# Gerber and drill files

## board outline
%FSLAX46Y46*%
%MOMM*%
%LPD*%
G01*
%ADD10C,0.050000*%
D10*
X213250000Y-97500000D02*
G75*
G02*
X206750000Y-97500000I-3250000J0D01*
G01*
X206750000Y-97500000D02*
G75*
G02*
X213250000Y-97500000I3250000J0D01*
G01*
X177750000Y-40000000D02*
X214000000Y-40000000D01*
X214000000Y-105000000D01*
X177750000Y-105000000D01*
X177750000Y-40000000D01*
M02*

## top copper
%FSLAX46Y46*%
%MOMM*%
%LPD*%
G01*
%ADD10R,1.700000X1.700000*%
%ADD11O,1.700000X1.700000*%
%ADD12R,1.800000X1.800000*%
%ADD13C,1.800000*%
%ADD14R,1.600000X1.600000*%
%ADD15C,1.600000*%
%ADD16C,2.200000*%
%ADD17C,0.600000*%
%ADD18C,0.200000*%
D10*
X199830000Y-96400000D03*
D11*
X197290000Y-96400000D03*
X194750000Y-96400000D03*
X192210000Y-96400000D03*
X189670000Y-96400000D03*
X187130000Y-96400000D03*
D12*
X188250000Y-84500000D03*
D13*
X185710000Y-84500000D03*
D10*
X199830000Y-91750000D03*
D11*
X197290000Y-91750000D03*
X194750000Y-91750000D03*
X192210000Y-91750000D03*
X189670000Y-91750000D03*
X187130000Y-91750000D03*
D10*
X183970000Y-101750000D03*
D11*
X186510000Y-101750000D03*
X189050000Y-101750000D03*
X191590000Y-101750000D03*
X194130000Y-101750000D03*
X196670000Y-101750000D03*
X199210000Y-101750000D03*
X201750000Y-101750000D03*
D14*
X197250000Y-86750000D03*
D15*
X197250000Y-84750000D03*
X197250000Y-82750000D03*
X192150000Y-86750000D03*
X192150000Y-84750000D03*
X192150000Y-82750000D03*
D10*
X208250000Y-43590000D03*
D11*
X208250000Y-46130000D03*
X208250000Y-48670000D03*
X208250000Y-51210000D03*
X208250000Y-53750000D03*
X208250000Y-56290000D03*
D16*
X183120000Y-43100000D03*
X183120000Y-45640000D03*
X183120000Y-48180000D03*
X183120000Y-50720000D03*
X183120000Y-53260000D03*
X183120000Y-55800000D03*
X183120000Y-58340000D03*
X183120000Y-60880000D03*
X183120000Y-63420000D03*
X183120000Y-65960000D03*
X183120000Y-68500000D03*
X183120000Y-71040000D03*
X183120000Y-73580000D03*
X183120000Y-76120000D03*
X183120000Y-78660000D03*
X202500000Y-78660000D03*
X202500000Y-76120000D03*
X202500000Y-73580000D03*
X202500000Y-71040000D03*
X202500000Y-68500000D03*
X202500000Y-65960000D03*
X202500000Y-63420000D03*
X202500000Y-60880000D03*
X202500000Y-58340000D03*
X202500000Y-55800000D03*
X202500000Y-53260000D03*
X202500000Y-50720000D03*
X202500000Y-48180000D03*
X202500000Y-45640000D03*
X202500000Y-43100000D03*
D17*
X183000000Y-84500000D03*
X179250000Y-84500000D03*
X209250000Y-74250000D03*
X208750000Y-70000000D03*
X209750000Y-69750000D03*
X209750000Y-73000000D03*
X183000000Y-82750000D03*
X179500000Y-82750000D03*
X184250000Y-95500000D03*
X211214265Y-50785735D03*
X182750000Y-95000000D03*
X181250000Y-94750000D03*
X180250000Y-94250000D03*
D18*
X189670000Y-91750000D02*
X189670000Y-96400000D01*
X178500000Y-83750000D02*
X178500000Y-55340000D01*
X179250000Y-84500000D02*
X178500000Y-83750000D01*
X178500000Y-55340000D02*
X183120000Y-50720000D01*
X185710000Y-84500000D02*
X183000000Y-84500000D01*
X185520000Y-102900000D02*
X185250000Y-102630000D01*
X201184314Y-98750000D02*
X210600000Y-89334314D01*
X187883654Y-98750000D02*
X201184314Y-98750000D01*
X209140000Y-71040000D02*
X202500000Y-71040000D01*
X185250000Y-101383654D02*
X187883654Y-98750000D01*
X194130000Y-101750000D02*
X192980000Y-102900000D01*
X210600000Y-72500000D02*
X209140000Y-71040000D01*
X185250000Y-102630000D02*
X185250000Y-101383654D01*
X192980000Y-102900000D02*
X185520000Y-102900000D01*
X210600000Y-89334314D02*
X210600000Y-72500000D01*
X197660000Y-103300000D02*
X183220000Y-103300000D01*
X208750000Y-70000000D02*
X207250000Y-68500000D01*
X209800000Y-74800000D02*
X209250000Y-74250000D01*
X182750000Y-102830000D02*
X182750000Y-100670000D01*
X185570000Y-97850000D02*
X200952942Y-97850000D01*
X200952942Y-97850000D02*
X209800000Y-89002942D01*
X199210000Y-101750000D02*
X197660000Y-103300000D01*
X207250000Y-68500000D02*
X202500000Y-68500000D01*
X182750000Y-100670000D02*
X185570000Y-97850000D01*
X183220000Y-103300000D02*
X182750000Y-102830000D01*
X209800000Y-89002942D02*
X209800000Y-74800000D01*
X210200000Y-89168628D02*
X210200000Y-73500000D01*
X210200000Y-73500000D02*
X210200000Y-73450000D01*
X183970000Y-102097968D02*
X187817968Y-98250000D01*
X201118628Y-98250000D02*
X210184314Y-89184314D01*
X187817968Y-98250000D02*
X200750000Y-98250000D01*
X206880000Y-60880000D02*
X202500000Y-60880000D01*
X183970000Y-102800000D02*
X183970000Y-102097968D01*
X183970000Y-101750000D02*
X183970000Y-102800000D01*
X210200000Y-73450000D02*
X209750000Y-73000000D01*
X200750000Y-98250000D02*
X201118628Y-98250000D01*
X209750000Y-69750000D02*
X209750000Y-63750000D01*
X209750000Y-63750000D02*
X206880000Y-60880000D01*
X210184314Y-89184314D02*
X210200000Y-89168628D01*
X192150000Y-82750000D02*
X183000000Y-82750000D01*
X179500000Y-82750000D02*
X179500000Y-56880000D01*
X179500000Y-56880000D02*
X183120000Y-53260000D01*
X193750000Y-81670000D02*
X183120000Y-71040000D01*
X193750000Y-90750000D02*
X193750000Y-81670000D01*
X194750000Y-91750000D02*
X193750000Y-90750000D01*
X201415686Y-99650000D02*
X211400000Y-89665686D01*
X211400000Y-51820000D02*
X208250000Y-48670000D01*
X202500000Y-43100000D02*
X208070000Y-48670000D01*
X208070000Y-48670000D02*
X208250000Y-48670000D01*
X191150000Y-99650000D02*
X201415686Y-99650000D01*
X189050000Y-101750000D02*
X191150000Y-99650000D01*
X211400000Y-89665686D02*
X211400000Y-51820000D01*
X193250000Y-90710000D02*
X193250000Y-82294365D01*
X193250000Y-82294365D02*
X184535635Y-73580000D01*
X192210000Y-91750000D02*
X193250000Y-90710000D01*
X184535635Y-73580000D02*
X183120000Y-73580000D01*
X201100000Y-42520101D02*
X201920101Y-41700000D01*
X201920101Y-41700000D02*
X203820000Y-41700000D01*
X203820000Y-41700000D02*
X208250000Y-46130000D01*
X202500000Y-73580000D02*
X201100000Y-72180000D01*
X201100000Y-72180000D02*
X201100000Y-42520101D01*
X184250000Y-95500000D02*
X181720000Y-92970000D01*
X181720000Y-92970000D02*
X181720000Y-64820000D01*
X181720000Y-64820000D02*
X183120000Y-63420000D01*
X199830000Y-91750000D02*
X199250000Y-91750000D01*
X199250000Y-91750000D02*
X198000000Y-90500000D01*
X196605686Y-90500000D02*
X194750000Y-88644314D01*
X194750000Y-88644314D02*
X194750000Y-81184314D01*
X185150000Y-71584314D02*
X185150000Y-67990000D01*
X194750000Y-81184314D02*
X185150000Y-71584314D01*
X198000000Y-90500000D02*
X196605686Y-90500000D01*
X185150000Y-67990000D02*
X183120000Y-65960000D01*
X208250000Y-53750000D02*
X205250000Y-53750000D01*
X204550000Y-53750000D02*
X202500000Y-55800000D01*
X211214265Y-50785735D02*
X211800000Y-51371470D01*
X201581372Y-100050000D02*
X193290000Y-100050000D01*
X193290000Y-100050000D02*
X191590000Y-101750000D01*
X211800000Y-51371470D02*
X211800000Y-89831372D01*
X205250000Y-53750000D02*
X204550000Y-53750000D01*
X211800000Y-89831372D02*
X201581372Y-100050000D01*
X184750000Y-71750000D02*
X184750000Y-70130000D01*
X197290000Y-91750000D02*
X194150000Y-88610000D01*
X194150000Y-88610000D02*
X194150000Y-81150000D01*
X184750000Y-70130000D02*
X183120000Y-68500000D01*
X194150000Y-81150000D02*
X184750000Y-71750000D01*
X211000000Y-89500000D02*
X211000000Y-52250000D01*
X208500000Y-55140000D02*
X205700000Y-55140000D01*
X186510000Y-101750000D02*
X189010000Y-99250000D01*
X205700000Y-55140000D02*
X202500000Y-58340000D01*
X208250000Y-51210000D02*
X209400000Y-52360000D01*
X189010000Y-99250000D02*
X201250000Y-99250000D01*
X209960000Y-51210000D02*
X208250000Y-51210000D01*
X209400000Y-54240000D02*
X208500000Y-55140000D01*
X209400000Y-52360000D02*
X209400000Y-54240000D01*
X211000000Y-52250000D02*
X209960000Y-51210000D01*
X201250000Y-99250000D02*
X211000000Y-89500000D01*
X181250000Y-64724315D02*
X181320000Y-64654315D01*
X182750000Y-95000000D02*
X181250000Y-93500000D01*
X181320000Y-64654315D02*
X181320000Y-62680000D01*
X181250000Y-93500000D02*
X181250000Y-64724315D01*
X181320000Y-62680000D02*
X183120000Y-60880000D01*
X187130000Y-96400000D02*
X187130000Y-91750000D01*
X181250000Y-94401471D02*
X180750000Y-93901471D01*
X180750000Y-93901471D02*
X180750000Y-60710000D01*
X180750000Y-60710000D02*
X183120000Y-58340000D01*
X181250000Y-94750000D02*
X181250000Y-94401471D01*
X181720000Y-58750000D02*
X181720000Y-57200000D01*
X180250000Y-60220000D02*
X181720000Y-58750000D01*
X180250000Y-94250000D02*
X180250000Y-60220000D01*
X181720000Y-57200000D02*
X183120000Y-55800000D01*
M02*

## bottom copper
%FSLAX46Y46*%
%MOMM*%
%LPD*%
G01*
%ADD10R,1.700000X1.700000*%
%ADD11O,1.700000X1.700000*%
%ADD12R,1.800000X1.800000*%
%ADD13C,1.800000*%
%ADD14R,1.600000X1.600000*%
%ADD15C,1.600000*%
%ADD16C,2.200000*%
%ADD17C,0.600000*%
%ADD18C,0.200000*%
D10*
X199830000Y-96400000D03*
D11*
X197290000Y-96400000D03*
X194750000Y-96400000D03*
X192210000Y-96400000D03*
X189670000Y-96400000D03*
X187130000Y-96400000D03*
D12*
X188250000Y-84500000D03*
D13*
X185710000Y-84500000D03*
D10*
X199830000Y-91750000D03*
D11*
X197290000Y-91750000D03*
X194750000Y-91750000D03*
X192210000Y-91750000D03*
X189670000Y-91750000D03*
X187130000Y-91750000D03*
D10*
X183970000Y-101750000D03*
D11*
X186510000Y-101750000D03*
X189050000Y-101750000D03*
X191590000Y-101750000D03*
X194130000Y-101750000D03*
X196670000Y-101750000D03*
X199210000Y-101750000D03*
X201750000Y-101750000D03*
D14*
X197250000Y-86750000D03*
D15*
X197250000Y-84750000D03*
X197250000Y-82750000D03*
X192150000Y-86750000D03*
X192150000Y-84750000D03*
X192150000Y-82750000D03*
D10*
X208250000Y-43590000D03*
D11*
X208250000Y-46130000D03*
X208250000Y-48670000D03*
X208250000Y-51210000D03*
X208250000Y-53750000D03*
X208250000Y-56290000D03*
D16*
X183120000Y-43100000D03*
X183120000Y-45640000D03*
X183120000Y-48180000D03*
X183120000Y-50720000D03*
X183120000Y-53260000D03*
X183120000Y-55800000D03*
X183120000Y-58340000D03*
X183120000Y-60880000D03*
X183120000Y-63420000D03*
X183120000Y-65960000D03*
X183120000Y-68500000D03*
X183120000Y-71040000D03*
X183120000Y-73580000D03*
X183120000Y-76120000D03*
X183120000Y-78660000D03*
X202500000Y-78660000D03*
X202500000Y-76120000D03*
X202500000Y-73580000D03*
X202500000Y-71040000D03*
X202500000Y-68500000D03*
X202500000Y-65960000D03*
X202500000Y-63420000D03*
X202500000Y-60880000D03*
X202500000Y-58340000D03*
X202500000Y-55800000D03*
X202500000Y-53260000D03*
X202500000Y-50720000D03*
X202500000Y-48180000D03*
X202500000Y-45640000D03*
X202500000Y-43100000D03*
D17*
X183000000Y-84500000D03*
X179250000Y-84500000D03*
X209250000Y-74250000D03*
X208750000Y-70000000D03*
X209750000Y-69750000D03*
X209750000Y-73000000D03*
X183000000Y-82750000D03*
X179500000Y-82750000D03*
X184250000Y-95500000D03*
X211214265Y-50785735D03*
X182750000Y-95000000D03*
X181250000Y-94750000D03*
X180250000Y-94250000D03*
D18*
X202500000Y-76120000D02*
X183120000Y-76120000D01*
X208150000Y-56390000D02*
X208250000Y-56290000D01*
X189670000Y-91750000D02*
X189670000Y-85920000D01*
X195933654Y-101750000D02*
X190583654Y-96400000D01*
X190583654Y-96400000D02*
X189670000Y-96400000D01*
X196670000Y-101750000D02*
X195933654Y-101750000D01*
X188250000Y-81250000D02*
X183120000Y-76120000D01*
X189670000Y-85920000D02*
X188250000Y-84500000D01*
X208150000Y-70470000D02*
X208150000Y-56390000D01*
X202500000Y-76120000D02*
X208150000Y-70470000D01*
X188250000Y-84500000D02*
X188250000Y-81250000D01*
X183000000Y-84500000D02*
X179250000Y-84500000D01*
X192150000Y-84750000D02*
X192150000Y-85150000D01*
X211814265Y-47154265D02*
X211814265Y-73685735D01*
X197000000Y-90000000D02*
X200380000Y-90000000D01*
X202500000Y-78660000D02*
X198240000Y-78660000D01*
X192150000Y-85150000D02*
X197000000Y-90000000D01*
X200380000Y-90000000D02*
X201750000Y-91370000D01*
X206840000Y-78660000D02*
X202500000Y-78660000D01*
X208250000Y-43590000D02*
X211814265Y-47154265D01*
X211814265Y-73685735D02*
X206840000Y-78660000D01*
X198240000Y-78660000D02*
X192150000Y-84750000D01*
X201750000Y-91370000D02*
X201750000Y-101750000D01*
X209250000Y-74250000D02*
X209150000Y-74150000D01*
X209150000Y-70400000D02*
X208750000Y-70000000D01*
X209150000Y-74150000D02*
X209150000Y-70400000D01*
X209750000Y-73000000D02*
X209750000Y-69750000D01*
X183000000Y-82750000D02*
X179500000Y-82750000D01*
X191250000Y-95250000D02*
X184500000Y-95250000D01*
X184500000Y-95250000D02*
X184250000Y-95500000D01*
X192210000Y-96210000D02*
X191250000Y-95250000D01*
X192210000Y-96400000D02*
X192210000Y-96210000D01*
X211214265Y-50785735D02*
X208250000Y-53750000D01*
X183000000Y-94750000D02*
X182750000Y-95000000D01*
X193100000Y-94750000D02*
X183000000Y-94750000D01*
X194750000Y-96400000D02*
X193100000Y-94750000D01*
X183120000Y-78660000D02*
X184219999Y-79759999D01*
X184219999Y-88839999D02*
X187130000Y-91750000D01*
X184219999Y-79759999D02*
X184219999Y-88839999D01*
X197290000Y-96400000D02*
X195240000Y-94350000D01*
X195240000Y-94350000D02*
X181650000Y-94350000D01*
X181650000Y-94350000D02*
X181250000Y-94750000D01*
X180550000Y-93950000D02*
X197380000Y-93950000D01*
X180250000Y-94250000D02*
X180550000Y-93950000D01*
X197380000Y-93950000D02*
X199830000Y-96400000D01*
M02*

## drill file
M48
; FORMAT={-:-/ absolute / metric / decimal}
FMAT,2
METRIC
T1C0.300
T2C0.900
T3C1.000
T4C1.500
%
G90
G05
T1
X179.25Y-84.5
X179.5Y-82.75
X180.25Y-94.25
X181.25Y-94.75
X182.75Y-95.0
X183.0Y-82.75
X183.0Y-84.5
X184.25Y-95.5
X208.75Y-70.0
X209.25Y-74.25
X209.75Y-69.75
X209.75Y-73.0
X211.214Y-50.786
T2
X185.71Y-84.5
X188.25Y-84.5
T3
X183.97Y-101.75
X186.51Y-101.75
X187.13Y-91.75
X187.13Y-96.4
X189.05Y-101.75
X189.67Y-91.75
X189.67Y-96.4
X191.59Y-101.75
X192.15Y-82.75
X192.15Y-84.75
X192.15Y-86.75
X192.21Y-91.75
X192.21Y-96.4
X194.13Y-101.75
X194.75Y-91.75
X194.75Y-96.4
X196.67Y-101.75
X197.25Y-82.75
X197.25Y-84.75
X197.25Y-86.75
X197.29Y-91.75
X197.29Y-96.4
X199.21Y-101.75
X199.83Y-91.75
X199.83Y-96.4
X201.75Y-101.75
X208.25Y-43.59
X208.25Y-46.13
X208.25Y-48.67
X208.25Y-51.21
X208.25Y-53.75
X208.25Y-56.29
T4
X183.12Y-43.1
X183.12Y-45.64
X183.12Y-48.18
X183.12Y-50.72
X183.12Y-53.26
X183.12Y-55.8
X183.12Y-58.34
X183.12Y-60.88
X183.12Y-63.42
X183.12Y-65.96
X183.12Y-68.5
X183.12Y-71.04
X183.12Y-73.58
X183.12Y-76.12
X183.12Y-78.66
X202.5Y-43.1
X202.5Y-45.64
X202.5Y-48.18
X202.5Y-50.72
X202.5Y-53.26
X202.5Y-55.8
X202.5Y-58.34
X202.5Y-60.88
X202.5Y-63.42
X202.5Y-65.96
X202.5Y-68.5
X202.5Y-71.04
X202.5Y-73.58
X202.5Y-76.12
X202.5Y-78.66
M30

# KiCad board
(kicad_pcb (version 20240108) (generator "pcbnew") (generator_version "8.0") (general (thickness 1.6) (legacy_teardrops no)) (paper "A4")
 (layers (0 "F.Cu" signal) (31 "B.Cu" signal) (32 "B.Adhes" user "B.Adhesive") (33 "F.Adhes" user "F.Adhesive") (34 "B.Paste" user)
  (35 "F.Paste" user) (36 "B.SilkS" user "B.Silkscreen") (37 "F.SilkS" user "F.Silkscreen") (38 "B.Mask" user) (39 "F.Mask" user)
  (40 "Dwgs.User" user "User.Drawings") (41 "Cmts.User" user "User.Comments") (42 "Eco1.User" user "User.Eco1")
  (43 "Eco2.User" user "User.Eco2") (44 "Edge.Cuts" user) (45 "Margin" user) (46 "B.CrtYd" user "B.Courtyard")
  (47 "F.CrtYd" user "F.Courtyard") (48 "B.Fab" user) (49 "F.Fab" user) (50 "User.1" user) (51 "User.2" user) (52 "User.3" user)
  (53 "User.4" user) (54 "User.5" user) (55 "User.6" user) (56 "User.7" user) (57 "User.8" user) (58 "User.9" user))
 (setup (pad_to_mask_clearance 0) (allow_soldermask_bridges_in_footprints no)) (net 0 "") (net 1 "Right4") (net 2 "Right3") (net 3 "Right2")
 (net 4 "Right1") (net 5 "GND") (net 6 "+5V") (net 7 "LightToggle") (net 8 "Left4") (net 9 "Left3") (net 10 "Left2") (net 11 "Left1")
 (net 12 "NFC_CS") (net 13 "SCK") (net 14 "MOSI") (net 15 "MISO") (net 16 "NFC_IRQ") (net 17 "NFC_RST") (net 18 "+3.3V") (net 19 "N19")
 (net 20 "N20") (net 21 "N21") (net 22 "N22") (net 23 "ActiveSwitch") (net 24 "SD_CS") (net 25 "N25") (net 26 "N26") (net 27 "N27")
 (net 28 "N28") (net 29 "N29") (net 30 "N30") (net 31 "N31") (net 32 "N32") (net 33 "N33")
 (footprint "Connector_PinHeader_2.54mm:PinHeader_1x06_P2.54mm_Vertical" (layer "F.Cu") (at 199.83 96.4 -90)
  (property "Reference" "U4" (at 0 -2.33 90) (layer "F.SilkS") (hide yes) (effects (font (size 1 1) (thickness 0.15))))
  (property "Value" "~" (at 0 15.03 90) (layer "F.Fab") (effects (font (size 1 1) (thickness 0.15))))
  (pad "1" thru_hole rect (at 0 0 270) (size 1.7 1.7) (drill 1) (layers "*.Cu" "*.Mask") (remove_unused_layers no) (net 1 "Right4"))
  (pad "2" thru_hole oval (at 0 2.54 270) (size 1.7 1.7) (drill 1) (layers "*.Cu" "*.Mask") (remove_unused_layers no) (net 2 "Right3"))
  (pad "3" thru_hole oval (at 0 5.08 270) (size 1.7 1.7) (drill 1) (layers "*.Cu" "*.Mask") (remove_unused_layers no) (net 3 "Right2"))
  (pad "4" thru_hole oval (at 0 7.62 270) (size 1.7 1.7) (drill 1) (layers "*.Cu" "*.Mask") (remove_unused_layers no) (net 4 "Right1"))
  (pad "5" thru_hole oval (at 0 10.16 270) (size 1.7 1.7) (drill 1) (layers "*.Cu" "*.Mask") (remove_unused_layers no) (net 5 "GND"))
  (pad "6" thru_hole oval (at 0 12.7 270) (size 1.7 1.7) (drill 1) (layers "*.Cu" "*.Mask") (remove_unused_layers no) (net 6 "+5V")))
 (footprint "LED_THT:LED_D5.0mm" (layer "F.Cu") (at 188.25 84.5 180)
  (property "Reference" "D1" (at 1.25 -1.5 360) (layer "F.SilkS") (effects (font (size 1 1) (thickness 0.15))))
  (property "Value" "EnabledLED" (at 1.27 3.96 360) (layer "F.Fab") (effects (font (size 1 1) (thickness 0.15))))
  (pad "1" thru_hole rect (at 0 0 180) (size 1.8 1.8) (drill 0.9) (layers "*.Cu" "*.Mask") (remove_unused_layers no) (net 5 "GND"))
  (pad "2" thru_hole circle (at 2.54 0 180) (size 1.8 1.8) (drill 0.9) (layers "*.Cu" "*.Mask") (remove_unused_layers no)
   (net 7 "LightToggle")))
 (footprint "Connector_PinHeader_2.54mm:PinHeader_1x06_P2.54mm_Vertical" (layer "F.Cu") (at 199.83 91.75 -90)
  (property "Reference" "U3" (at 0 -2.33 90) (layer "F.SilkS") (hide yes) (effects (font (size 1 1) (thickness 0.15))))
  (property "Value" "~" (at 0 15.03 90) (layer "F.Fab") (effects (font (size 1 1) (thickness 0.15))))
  (pad "1" thru_hole rect (at 0 0 270) (size 1.7 1.7) (drill 1) (layers "*.Cu" "*.Mask") (remove_unused_layers no) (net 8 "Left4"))
  (pad "2" thru_hole oval (at 0 2.54 270) (size 1.7 1.7) (drill 1) (layers "*.Cu" "*.Mask") (remove_unused_layers no) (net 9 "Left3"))
  (pad "3" thru_hole oval (at 0 5.08 270) (size 1.7 1.7) (drill 1) (layers "*.Cu" "*.Mask") (remove_unused_layers no) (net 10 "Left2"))
  (pad "4" thru_hole oval (at 0 7.62 270) (size 1.7 1.7) (drill 1) (layers "*.Cu" "*.Mask") (remove_unused_layers no) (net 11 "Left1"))
  (pad "5" thru_hole oval (at 0 10.16 270) (size 1.7 1.7) (drill 1) (layers "*.Cu" "*.Mask") (remove_unused_layers no) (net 5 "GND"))
  (pad "6" thru_hole oval (at 0 12.7 270) (size 1.7 1.7) (drill 1) (layers "*.Cu" "*.Mask") (remove_unused_layers no) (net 6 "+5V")))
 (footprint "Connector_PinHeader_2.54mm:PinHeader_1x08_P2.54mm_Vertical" (layer "F.Cu") (at 183.97 101.75 90)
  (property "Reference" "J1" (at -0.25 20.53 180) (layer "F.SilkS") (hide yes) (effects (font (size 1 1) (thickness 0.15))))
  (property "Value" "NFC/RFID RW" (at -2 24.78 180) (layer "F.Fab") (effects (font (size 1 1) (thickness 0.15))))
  (pad "1" thru_hole rect (at 0 0 90) (size 1.7 1.7) (drill 1) (layers "*.Cu" "*.Mask") (remove_unused_layers no) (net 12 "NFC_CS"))
  (pad "2" thru_hole oval (at 0 2.54 90) (size 1.7 1.7) (drill 1) (layers "*.Cu" "*.Mask") (remove_unused_layers no) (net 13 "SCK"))
  (pad "3" thru_hole oval (at 0 5.08 90) (size 1.7 1.7) (drill 1) (layers "*.Cu" "*.Mask") (remove_unused_layers no) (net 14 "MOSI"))
  (pad "4" thru_hole oval (at 0 7.62 90) (size 1.7 1.7) (drill 1) (layers "*.Cu" "*.Mask") (remove_unused_layers no) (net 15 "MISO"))
  (pad "5" thru_hole oval (at 0 10.16 90) (size 1.7 1.7) (drill 1) (layers "*.Cu" "*.Mask") (remove_unused_layers no) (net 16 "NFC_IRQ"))
  (pad "6" thru_hole oval (at 0 12.7 90) (size 1.7 1.7) (drill 1) (layers "*.Cu" "*.Mask") (remove_unused_layers no) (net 5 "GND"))
  (pad "7" thru_hole oval (at 0 15.24 90) (size 1.7 1.7) (drill 1) (layers "*.Cu" "*.Mask") (remove_unused_layers no) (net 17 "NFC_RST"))
  (pad "8" thru_hole oval (at 0 17.78 90) (size 1.7 1.7) (drill 1) (layers "*.Cu" "*.Mask") (remove_unused_layers no) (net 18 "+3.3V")))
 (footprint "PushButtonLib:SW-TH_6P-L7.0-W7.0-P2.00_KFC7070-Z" (layer "F.Cu") (at 194.7 84.75)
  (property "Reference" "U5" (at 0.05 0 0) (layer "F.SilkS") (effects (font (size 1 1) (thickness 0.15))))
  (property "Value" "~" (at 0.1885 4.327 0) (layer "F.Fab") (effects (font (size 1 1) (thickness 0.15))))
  (pad "1" thru_hole rect (at 2.55 2 270) (size 1.6 1.6) (drill 1) (layers "*.Cu" "*.Mask") (remove_unused_layers no) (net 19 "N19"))
  (pad "2" thru_hole circle (at 2.55 0 270) (size 1.6 1.6) (drill 1) (layers "*.Cu" "*.Mask") (remove_unused_layers no) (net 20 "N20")
   (thermal_bridge_angle 90))
  (pad "3" thru_hole circle (at 2.55 -2 270) (size 1.6 1.6) (drill 1) (layers "*.Cu" "*.Mask") (remove_unused_layers no) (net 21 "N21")
   (thermal_bridge_angle 90))
  (pad "4" thru_hole circle (at -2.55 2 270) (size 1.6 1.6) (drill 1) (layers "*.Cu" "*.Mask") (remove_unused_layers no) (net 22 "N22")
   (thermal_bridge_angle 90))
  (pad "5" thru_hole circle (at -2.55 0 270) (size 1.6 1.6) (drill 1) (layers "*.Cu" "*.Mask") (remove_unused_layers no) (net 18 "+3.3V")
   (thermal_bridge_angle 90))
  (pad "6" thru_hole circle (at -2.55 -2 270) (size 1.6 1.6) (drill 1) (layers "*.Cu" "*.Mask") (remove_unused_layers no)
   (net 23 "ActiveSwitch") (thermal_bridge_angle 90)))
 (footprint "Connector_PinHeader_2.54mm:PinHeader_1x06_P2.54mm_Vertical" (layer "F.Cu") (at 208.25 43.59)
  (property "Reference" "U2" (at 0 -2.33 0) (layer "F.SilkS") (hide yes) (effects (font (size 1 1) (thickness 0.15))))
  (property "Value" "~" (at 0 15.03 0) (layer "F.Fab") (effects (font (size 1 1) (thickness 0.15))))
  (pad "1" thru_hole rect (at 0 0) (size 1.7 1.7) (drill 1) (layers "*.Cu" "*.Mask") (remove_unused_layers no) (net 18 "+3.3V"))
  (pad "2" thru_hole oval (at 0 2.54) (size 1.7 1.7) (drill 1) (layers "*.Cu" "*.Mask") (remove_unused_layers no) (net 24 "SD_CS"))
  (pad "3" thru_hole oval (at 0 5.08) (size 1.7 1.7) (drill 1) (layers "*.Cu" "*.Mask") (remove_unused_layers no) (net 14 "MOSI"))
  (pad "4" thru_hole oval (at 0 7.62) (size 1.7 1.7) (drill 1) (layers "*.Cu" "*.Mask") (remove_unused_layers no) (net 13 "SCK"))
  (pad "5" thru_hole oval (at 0 10.16) (size 1.7 1.7) (drill 1) (layers "*.Cu" "*.Mask") (remove_unused_layers no) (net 15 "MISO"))
  (pad "6" thru_hole oval (at 0 12.7) (size 1.7 1.7) (drill 1) (layers "*.Cu" "*.Mask") (remove_unused_layers no) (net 5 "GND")))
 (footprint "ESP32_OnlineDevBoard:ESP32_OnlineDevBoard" (layer "F.Cu") (at 192.901386 67.23 -90)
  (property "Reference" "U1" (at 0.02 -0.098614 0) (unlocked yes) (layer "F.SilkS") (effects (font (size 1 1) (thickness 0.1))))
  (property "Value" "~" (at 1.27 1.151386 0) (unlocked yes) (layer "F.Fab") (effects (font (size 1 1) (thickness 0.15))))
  (pad "1" thru_hole circle (at -24.13 9.781386 270) (size 2.2 2.2) (drill 1.5) (layers "*.Cu" "*.Mask") (remove_unused_layers no)
   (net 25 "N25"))
  (pad "2" thru_hole circle (at -21.59 9.781386 270) (size 2.2 2.2) (drill 1.5) (layers "*.Cu" "*.Mask") (remove_unused_layers no)
   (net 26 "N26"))
  (pad "3" thru_hole circle (at -19.05 9.781386 270) (size 2.2 2.2) (drill 1.5) (layers "*.Cu" "*.Mask") (remove_unused_layers no)
   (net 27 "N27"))
  (pad "4" thru_hole circle (at -16.51 9.781386 270) (size 2.2 2.2) (drill 1.5) (layers "*.Cu" "*.Mask") (remove_unused_layers no)
   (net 7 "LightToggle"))
  (pad "5" thru_hole circle (at -13.97 9.781386 270) (size 2.2 2.2) (drill 1.5) (layers "*.Cu" "*.Mask") (remove_unused_layers no)
   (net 23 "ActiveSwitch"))
  (pad "6" thru_hole circle (at -11.43 9.781386 270) (size 2.2 2.2) (drill 1.5) (layers "*.Cu" "*.Mask") (remove_unused_layers no)
   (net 1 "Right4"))
  (pad "7" thru_hole circle (at -8.89 9.781386 270) (size 2.2 2.2) (drill 1.5) (layers "*.Cu" "*.Mask") (remove_unused_layers no)
   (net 2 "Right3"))
  (pad "8" thru_hole circle (at -6.35 9.781386 270) (size 2.2 2.2) (drill 1.5) (layers "*.Cu" "*.Mask") (remove_unused_layers no)
   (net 3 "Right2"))
  (pad "9" thru_hole circle (at -3.81 9.781386 270) (size 2.2 2.2) (drill 1.5) (layers "*.Cu" "*.Mask") (remove_unused_layers no)
   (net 4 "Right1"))
  (pad "10" thru_hole circle (at -1.27 9.781386 270) (size 2.2 2.2) (drill 1.5) (layers "*.Cu" "*.Mask") (remove_unused_layers no)
   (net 8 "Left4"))
  (pad "11" thru_hole circle (at 1.27 9.781386 270) (size 2.2 2.2) (drill 1.5) (layers "*.Cu" "*.Mask") (remove_unused_layers no)
   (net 9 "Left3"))
  (pad "12" thru_hole circle (at 3.81 9.781386 270) (size 2.2 2.2) (drill 1.5) (layers "*.Cu" "*.Mask") (remove_unused_layers no)
   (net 10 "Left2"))
  (pad "13" thru_hole circle (at 6.35 9.781386 270) (size 2.2 2.2) (drill 1.5) (layers "*.Cu" "*.Mask") (remove_unused_layers no)
   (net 11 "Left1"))
  (pad "14" thru_hole circle (at 8.89 9.781386 270) (size 2.2 2.2) (drill 1.5) (layers "*.Cu" "*.Mask") (remove_unused_layers no)
   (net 5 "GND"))
  (pad "15" thru_hole circle (at 11.43 9.781386 270) (size 2.2 2.2) (drill 1.5) (layers "*.Cu" "*.Mask") (remove_unused_layers no)
   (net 6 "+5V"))
  (pad "16" thru_hole circle (at 11.43 -9.598614 270) (size 2.2 2.2) (drill 1.5) (layers "*.Cu" "*.Mask") (remove_unused_layers no)
   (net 18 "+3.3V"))
  (pad "17" thru_hole circle (at 8.89 -9.598614 270) (size 2.2 2.2) (drill 1.5) (layers "*.Cu" "*.Mask") (remove_unused_layers no)
   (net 5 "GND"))
  (pad "18" thru_hole circle (at 6.35 -9.598614 270) (size 2.2 2.2) (drill 1.5) (layers "*.Cu" "*.Mask") (remove_unused_layers no)
   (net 24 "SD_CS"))
  (pad "19" thru_hole circle (at 3.81 -9.598614 270) (size 2.2 2.2) (drill 1.5) (layers "*.Cu" "*.Mask") (remove_unused_layers no)
   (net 16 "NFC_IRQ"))
  (pad "20" thru_hole circle (at 1.27 -9.598614 270) (size 2.2 2.2) (drill 1.5) (layers "*.Cu" "*.Mask") (remove_unused_layers no)
   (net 17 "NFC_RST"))
  (pad "21" thru_hole circle (at -1.27 -9.598614 270) (size 2.2 2.2) (drill 1.5) (layers "*.Cu" "*.Mask") (remove_unused_layers no)
   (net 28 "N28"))
  (pad "22" thru_hole circle (at -3.81 -9.598614 270) (size 2.2 2.2) (drill 1.5) (layers "*.Cu" "*.Mask") (remove_unused_layers no)
   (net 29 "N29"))
  (pad "23" thru_hole circle (at -6.35 -9.598614 270) (size 2.2 2.2) (drill 1.5) (layers "*.Cu" "*.Mask") (remove_unused_layers no)
   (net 12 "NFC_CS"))
  (pad "24" thru_hole circle (at -8.89 -9.598614 270) (size 2.2 2.2) (drill 1.5) (layers "*.Cu" "*.Mask") (remove_unused_layers no)
   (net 13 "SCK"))
  (pad "25" thru_hole circle (at -11.43 -9.598614 270) (size 2.2 2.2) (drill 1.5) (layers "*.Cu" "*.Mask") (remove_unused_layers no)
   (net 15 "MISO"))
  (pad "26" thru_hole circle (at -13.97 -9.598614 270) (size 2.2 2.2) (drill 1.5) (layers "*.Cu" "*.Mask") (remove_unused_layers no)
   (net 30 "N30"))
  (pad "27" thru_hole circle (at -16.51 -9.598614 270) (size 2.2 2.2) (drill 1.5) (layers "*.Cu" "*.Mask") (remove_unused_layers no)
   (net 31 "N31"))
  (pad "28" thru_hole circle (at -19.05 -9.598614 270) (size 2.2 2.2) (drill 1.5) (layers "*.Cu" "*.Mask") (remove_unused_layers no)
   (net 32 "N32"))
  (pad "29" thru_hole circle (at -21.59 -9.598614 270) (size 2.2 2.2) (drill 1.5) (layers "*.Cu" "*.Mask") (remove_unused_layers no)
   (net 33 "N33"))
  (pad "30" thru_hole circle (at -24.13 -9.598614 270) (size 2.2 2.2) (drill 1.5) (layers "*.Cu" "*.Mask") (remove_unused_layers no)
   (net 14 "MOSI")))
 (gr_circle (center 210 97.5) (end 213.25 97.5) (stroke (width 0.05) (type default)) (fill none) (layer "Edge.Cuts"))
 (gr_rect (start 177.75 40) (end 214 105) (stroke (width 0.05) (type default)) (fill none) (layer "Edge.Cuts"))
 (segment (start 189.67 91.75) (end 189.67 96.4) (width 0.2) (layer "F.Cu") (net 5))
 (segment (start 202.5 76.12) (end 183.12 76.12) (width 0.2) (layer "B.Cu") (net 5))
 (segment (start 208.15 56.39) (end 208.25 56.29) (width 0.2) (layer "B.Cu") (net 5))
 (segment (start 189.67 91.75) (end 189.67 85.92) (width 0.2) (layer "B.Cu") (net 5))
 (segment (start 195.933654 101.75) (end 190.583654 96.4) (width 0.2) (layer "B.Cu") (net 5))
 (segment (start 190.583654 96.4) (end 189.67 96.4) (width 0.2) (layer "B.Cu") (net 5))
 (segment (start 196.67 101.75) (end 195.933654 101.75) (width 0.2) (layer "B.Cu") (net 5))
 (segment (start 188.25 81.25) (end 183.12 76.12) (width 0.2) (layer "B.Cu") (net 5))
 (segment (start 189.67 85.92) (end 188.25 84.5) (width 0.2) (layer "B.Cu") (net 5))
 (segment (start 208.15 70.47) (end 208.15 56.39) (width 0.2) (layer "B.Cu") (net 5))
 (segment (start 202.5 76.12) (end 208.15 70.47) (width 0.2) (layer "B.Cu") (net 5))
 (segment (start 188.25 84.5) (end 188.25 81.25) (width 0.2) (layer "B.Cu") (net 5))
 (segment (start 178.5 83.75) (end 178.5 55.34) (width 0.2) (layer "F.Cu") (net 7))
 (segment (start 179.25 84.5) (end 178.5 83.75) (width 0.2) (layer "F.Cu") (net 7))
 (segment (start 178.5 55.34) (end 183.12 50.72) (width 0.2) (layer "F.Cu") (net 7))
 (segment (start 185.71 84.5) (end 183 84.5) (width 0.2) (layer "F.Cu") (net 7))
 (via (at 183 84.5) (size 0.6) (drill 0.3) (layers "F.Cu" "B.Cu") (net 7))
 (via (at 179.25 84.5) (size 0.6) (drill 0.3) (layers "F.Cu" "B.Cu") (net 7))
 (segment (start 183 84.5) (end 179.25 84.5) (width 0.2) (layer "B.Cu") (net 7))
 (segment (start 192.15 84.75) (end 192.15 85.15) (width 0.2) (layer "B.Cu") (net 18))
 (segment (start 211.814265 47.154265) (end 211.814265 73.685735) (width 0.2) (layer "B.Cu") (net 18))
 (segment (start 197 90) (end 200.38 90) (width 0.2) (layer "B.Cu") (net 18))
 (segment (start 202.5 78.66) (end 198.24 78.66) (width 0.2) (layer "B.Cu") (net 18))
 (segment (start 192.15 85.15) (end 197 90) (width 0.2) (layer "B.Cu") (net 18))
 (segment (start 200.38 90) (end 201.75 91.37) (width 0.2) (layer "B.Cu") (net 18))
 (segment (start 206.84 78.66) (end 202.5 78.66) (width 0.2) (layer "B.Cu") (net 18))
 (segment (start 208.25 43.59) (end 211.814265 47.154265) (width 0.2) (layer "B.Cu") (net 18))
 (segment (start 211.814265 73.685735) (end 206.84 78.66) (width 0.2) (layer "B.Cu") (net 18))
 (segment (start 198.24 78.66) (end 192.15 84.75) (width 0.2) (layer "B.Cu") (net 18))
 (segment (start 201.75 91.37) (end 201.75 101.75) (width 0.2) (layer "B.Cu") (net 18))
 (segment (start 185.52 102.9) (end 185.25 102.63) (width 0.2) (layer "F.Cu") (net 16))
 (segment (start 201.184314 98.75) (end 210.6 89.334314) (width 0.2) (layer "F.Cu") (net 16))
 (segment (start 187.883654 98.75) (end 201.184314 98.75) (width 0.2) (layer "F.Cu") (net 16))
 (segment (start 209.14 71.04) (end 202.5 71.04) (width 0.2) (layer "F.Cu") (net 16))
 (segment (start 185.25 101.383654) (end 187.883654 98.75) (width 0.2) (layer "F.Cu") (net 16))
 (segment (start 194.13 101.75) (end 192.98 102.9) (width 0.2) (layer "F.Cu") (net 16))
 (segment (start 210.6 72.5) (end 209.14 71.04) (width 0.2) (layer "F.Cu") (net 16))
 (segment (start 185.25 102.63) (end 185.25 101.383654) (width 0.2) (layer "F.Cu") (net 16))
 (segment (start 192.98 102.9) (end 185.52 102.9) (width 0.2) (layer "F.Cu") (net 16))
 (segment (start 210.6 89.334314) (end 210.6 72.5) (width 0.2) (layer "F.Cu") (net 16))
 (segment (start 197.66 103.3) (end 183.22 103.3) (width 0.2) (layer "F.Cu") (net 17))
 (segment (start 208.75 70) (end 207.25 68.5) (width 0.2) (layer "F.Cu") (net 17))
 (segment (start 209.8 74.8) (end 209.25 74.25) (width 0.2) (layer "F.Cu") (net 17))
 (segment (start 182.75 102.83) (end 182.75 100.67) (width 0.2) (layer "F.Cu") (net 17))
 (segment (start 185.57 97.85) (end 200.952942 97.85) (width 0.2) (layer "F.Cu") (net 17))
 (segment (start 200.952942 97.85) (end 209.8 89.002942) (width 0.2) (layer "F.Cu") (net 17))
 (segment (start 199.21 101.75) (end 197.66 103.3) (width 0.2) (layer "F.Cu") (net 17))
 (segment (start 207.25 68.5) (end 202.5 68.5) (width 0.2) (layer "F.Cu") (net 17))
 (segment (start 182.75 100.67) (end 185.57 97.85) (width 0.2) (layer "F.Cu") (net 17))
 (segment (start 183.22 103.3) (end 182.75 102.83) (width 0.2) (layer "F.Cu") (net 17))
 (segment (start 209.8 89.002942) (end 209.8 74.8) (width 0.2) (layer "F.Cu") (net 17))
 (via (at 209.25 74.25) (size 0.6) (drill 0.3) (layers "F.Cu" "B.Cu") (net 17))
 (via (at 208.75 70) (size 0.6) (drill 0.3) (layers "F.Cu" "B.Cu") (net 17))
 (segment (start 209.25 74.25) (end 209.15 74.15) (width 0.2) (layer "B.Cu") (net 17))
 (segment (start 209.15 70.4) (end 208.75 70) (width 0.2) (layer "B.Cu") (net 17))
 (segment (start 209.15 74.15) (end 209.15 70.4) (width 0.2) (layer "B.Cu") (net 17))
 (segment (start 210.2 89.168628) (end 210.2 73.5) (width 0.2) (layer "F.Cu") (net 12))
 (segment (start 210.2 73.5) (end 210.2 73.45) (width 0.2) (layer "F.Cu") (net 12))
 (segment (start 183.97 102.097968) (end 187.817968 98.25) (width 0.2) (layer "F.Cu") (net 12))
 (segment (start 201.118628 98.25) (end 210.184314 89.184314) (width 0.2) (layer "F.Cu") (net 12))
 (segment (start 187.817968 98.25) (end 200.75 98.25) (width 0.2) (layer "F.Cu") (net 12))
 (segment (start 206.88 60.88) (end 202.5 60.88) (width 0.2) (layer "F.Cu") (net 12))
 (segment (start 183.97 102.8) (end 183.97 102.097968) (width 0.2) (layer "F.Cu") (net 12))
 (segment (start 183.97 101.75) (end 183.97 102.8) (width 0.2) (layer "F.Cu") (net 12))
 (segment (start 210.2 73.45) (end 209.75 73) (width 0.2) (layer "F.Cu") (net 12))
 (segment (start 200.75 98.25) (end 201.118628 98.25) (width 0.2) (layer "F.Cu") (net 12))
 (segment (start 209.75 69.75) (end 209.75 63.75) (width 0.2) (layer "F.Cu") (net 12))
 (segment (start 209.75 63.75) (end 206.88 60.88) (width 0.2) (layer "F.Cu") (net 12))
 (segment (start 210.184314 89.184314) (end 210.2 89.168628) (width 0.2) (layer "F.Cu") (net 12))
 (via (at 209.75 69.75) (size 0.6) (drill 0.3) (layers "F.Cu" "B.Cu") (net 12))
 (via (at 209.75 73) (size 0.6) (drill 0.3) (layers "F.Cu" "B.Cu") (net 12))
 (segment (start 209.75 73) (end 209.75 69.75) (width 0.2) (layer "B.Cu") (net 12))
 (segment (start 192.15 82.75) (end 183 82.75) (width 0.2) (layer "F.Cu") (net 23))
 (segment (start 179.5 82.75) (end 179.5 56.88) (width 0.2) (layer "F.Cu") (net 23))
 (segment (start 179.5 56.88) (end 183.12 53.26) (width 0.2) (layer "F.Cu") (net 23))
 (via (at 183 82.75) (size 0.6) (drill 0.3) (layers "F.Cu" "B.Cu") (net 23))
 (via (at 179.5 82.75) (size 0.6) (drill 0.3) (layers "F.Cu" "B.Cu") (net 23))
 (segment (start 183 82.75) (end 179.5 82.75) (width 0.2) (layer "B.Cu") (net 23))
 (segment (start 193.75 81.67) (end 183.12 71.04) (width 0.2) (layer "F.Cu") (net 10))
 (segment (start 193.75 90.75) (end 193.75 81.67) (width 0.2) (layer "F.Cu") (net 10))
 (segment (start 194.75 91.75) (end 193.75 90.75) (width 0.2) (layer "F.Cu") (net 10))
 (segment (start 201.415686 99.65) (end 211.4 89.665686) (width 0.2) (layer "F.Cu") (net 14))
 (segment (start 211.4 51.82) (end 208.25 48.67) (width 0.2) (layer "F.Cu") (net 14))
 (segment (start 202.5 43.1) (end 208.07 48.67) (width 0.2) (layer "F.Cu") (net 14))
 (segment (start 208.07 48.67) (end 208.25 48.67) (width 0.2) (layer "F.Cu") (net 14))
 (segment (start 191.15 99.65) (end 201.415686 99.65) (width 0.2) (layer "F.Cu") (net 14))
 (segment (start 189.05 101.75) (end 191.15 99.65) (width 0.2) (layer "F.Cu") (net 14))
 (segment (start 211.4 89.665686) (end 211.4 51.82) (width 0.2) (layer "F.Cu") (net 14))
 (segment (start 193.25 90.71) (end 193.25 82.294365) (width 0.2) (layer "F.Cu") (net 11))
 (segment (start 193.25 82.294365) (end 184.535635 73.58) (width 0.2) (layer "F.Cu") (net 11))
 (segment (start 192.21 91.75) (end 193.25 90.71) (width 0.2) (layer "F.Cu") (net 11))
 (segment (start 184.535635 73.58) (end 183.12 73.58) (width 0.2) (layer "F.Cu") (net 11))
 (segment (start 201.1 42.520101) (end 201.920101 41.7) (width 0.2) (layer "F.Cu") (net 24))
 (segment (start 201.920101 41.7) (end 203.82 41.7) (width 0.2) (layer "F.Cu") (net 24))
 (segment (start 203.82 41.7) (end 208.25 46.13) (width 0.2) (layer "F.Cu") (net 24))
 (segment (start 202.5 73.58) (end 201.1 72.18) (width 0.2) (layer "F.Cu") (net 24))
 (segment (start 201.1 72.18) (end 201.1 42.520101) (width 0.2) (layer "F.Cu") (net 24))
 (segment (start 184.25 95.5) (end 181.72 92.97) (width 0.2) (layer "F.Cu") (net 4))
 (segment (start 181.72 92.97) (end 181.72 64.82) (width 0.2) (layer "F.Cu") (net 4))
 (segment (start 181.72 64.82) (end 183.12 63.42) (width 0.2) (layer "F.Cu") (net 4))
 (via (at 184.25 95.5) (size 0.6) (drill 0.3) (layers "F.Cu" "B.Cu") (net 4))
 (segment (start 191.25 95.25) (end 184.5 95.25) (width 0.2) (layer "B.Cu") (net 4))
 (segment (start 184.5 95.25) (end 184.25 95.5) (width 0.2) (layer "B.Cu") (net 4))
 (segment (start 192.21 96.21) (end 191.25 95.25) (width 0.2) (layer "B.Cu") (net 4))
 (segment (start 192.21 96.4) (end 192.21 96.21) (width 0.2) (layer "B.Cu") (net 4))
 (segment (start 199.83 91.75) (end 199.25 91.75) (width 0.2) (layer "F.Cu") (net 8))
 (segment (start 199.25 91.75) (end 198 90.5) (width 0.2) (layer "F.Cu") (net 8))
 (segment (start 196.605686 90.5) (end 194.75 88.644314) (width 0.2) (layer "F.Cu") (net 8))
 (segment (start 194.75 88.644314) (end 194.75 81.184314) (width 0.2) (layer "F.Cu") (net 8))
 (segment (start 185.15 71.584314) (end 185.15 67.99) (width 0.2) (layer "F.Cu") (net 8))
 (segment (start 194.75 81.184314) (end 185.15 71.584314) (width 0.2) (layer "F.Cu") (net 8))
 (segment (start 198 90.5) (end 196.605686 90.5) (width 0.2) (layer "F.Cu") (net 8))
 (segment (start 185.15 67.99) (end 183.12 65.96) (width 0.2) (layer "F.Cu") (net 8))
 (segment (start 208.25 53.75) (end 205.25 53.75) (width 0.2) (layer "F.Cu") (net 15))
 (segment (start 204.55 53.75) (end 202.5 55.8) (width 0.2) (layer "F.Cu") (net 15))
 (segment (start 211.214265 50.785735) (end 211.8 51.37147) (width 0.2) (layer "F.Cu") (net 15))
 (segment (start 201.581372 100.05) (end 193.29 100.05) (width 0.2) (layer "F.Cu") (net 15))
 (segment (start 193.29 100.05) (end 191.59 101.75) (width 0.2) (layer "F.Cu") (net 15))
 (segment (start 211.8 51.37147) (end 211.8 89.831372) (width 0.2) (layer "F.Cu") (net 15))
 (segment (start 205.25 53.75) (end 204.55 53.75) (width 0.2) (layer "F.Cu") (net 15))
 (segment (start 211.8 89.831372) (end 201.581372 100.05) (width 0.2) (layer "F.Cu") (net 15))
 (via (at 211.214265 50.785735) (size 0.6) (drill 0.3) (layers "F.Cu" "B.Cu") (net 15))
 (segment (start 211.214265 50.785735) (end 208.25 53.75) (width 0.2) (layer "B.Cu") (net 15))
 (segment (start 184.75 71.75) (end 184.75 70.13) (width 0.2) (layer "F.Cu") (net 9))
 (segment (start 197.29 91.75) (end 194.15 88.61) (width 0.2) (layer "F.Cu") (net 9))
 (segment (start 194.15 88.61) (end 194.15 81.15) (width 0.2) (layer "F.Cu") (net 9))
 (segment (start 184.75 70.13) (end 183.12 68.5) (width 0.2) (layer "F.Cu") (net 9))
 (segment (start 194.15 81.15) (end 184.75 71.75) (width 0.2) (layer "F.Cu") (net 9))
 (segment (start 211 89.5) (end 211 52.25) (width 0.2) (layer "F.Cu") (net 13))
 (segment (start 208.5 55.14) (end 205.7 55.14) (width 0.2) (layer "F.Cu") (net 13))
 (segment (start 186.51 101.75) (end 189.01 99.25) (width 0.2) (layer "F.Cu") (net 13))
 (segment (start 205.7 55.14) (end 202.5 58.34) (width 0.2) (layer "F.Cu") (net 13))
 (segment (start 208.25 51.21) (end 209.4 52.36) (width 0.2) (layer "F.Cu") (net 13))
 (segment (start 189.01 99.25) (end 201.25 99.25) (width 0.2) (layer "F.Cu") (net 13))
 (segment (start 209.96 51.21) (end 208.25 51.21) (width 0.2) (layer "F.Cu") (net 13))
 (segment (start 209.4 54.24) (end 208.5 55.14) (width 0.2) (layer "F.Cu") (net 13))
 (segment (start 209.4 52.36) (end 209.4 54.24) (width 0.2) (layer "F.Cu") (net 13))
 (segment (start 211 52.25) (end 209.96 51.21) (width 0.2) (layer "F.Cu") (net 13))
 (segment (start 201.25 99.25) (end 211 89.5) (width 0.2) (layer "F.Cu") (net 13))
 (segment (start 181.25 64.724315) (end 181.32 64.654315) (width 0.2) (layer "F.Cu") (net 3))
 (segment (start 182.75 95) (end 181.25 93.5) (width 0.2) (layer "F.Cu") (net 3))
 (segment (start 181.32 64.654315) (end 181.32 62.68) (width 0.2) (layer "F.Cu") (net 3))
 (segment (start 181.25 93.5) (end 181.25 64.724315) (width 0.2) (layer "F.Cu") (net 3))
 (segment (start 181.32 62.68) (end 183.12 60.88) (width 0.2) (layer "F.Cu") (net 3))
 (via (at 182.75 95) (size 0.6) (drill 0.3) (layers "F.Cu" "B.Cu") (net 3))
 (segment (start 183 94.75) (end 182.75 95) (width 0.2) (layer "B.Cu") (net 3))
 (segment (start 193.1 94.75) (end 183 94.75) (width 0.2) (layer "B.Cu") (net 3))
 (segment (start 194.75 96.4) (end 193.1 94.75) (width 0.2) (layer "B.Cu") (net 3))
 (segment (start 187.13 96.4) (end 187.13 91.75) (width 0.2) (layer "F.Cu") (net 6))
 (segment (start 183.12 78.66) (end 184.219999 79.759999) (width 0.2) (layer "B.Cu") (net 6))
 (segment (start 184.219999 88.839999) (end 187.13 91.75) (width 0.2) (layer "B.Cu") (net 6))
 (segment (start 184.219999 79.759999) (end 184.219999 88.839999) (width 0.2) (layer "B.Cu") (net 6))
 (segment (start 181.25 94.401471) (end 180.75 93.901471) (width 0.2) (layer "F.Cu") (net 2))
 (segment (start 180.75 93.901471) (end 180.75 60.71) (width 0.2) (layer "F.Cu") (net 2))
 (segment (start 180.75 60.71) (end 183.12 58.34) (width 0.2) (layer "F.Cu") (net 2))
 (segment (start 181.25 94.75) (end 181.25 94.401471) (width 0.2) (layer "F.Cu") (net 2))
 (via (at 181.25 94.75) (size 0.6) (drill 0.3) (layers "F.Cu" "B.Cu") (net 2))
 (segment (start 197.29 96.4) (end 195.24 94.35) (width 0.2) (layer "B.Cu") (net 2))
 (segment (start 195.24 94.35) (end 181.65 94.35) (width 0.2) (layer "B.Cu") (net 2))
 (segment (start 181.65 94.35) (end 181.25 94.75) (width 0.2) (layer "B.Cu") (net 2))
 (segment (start 181.72 58.75) (end 181.72 57.2) (width 0.2) (layer "F.Cu") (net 1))
 (segment (start 180.25 60.22) (end 181.72 58.75) (width 0.2) (layer "F.Cu") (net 1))
 (segment (start 180.25 94.25) (end 180.25 60.22) (width 0.2) (layer "F.Cu") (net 1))
 (segment (start 181.72 57.2) (end 183.12 55.8) (width 0.2) (layer "F.Cu") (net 1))
 (via (at 180.25 94.25) (size 0.6) (drill 0.3) (layers "F.Cu" "B.Cu") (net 1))
 (segment (start 180.55 93.95) (end 197.38 93.95) (width 0.2) (layer "B.Cu") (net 1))
 (segment (start 180.25 94.25) (end 180.55 93.95) (width 0.2) (layer "B.Cu") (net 1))
 (segment (start 197.38 93.95) (end 199.83 96.4) (width 0.2) (layer "B.Cu") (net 1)))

